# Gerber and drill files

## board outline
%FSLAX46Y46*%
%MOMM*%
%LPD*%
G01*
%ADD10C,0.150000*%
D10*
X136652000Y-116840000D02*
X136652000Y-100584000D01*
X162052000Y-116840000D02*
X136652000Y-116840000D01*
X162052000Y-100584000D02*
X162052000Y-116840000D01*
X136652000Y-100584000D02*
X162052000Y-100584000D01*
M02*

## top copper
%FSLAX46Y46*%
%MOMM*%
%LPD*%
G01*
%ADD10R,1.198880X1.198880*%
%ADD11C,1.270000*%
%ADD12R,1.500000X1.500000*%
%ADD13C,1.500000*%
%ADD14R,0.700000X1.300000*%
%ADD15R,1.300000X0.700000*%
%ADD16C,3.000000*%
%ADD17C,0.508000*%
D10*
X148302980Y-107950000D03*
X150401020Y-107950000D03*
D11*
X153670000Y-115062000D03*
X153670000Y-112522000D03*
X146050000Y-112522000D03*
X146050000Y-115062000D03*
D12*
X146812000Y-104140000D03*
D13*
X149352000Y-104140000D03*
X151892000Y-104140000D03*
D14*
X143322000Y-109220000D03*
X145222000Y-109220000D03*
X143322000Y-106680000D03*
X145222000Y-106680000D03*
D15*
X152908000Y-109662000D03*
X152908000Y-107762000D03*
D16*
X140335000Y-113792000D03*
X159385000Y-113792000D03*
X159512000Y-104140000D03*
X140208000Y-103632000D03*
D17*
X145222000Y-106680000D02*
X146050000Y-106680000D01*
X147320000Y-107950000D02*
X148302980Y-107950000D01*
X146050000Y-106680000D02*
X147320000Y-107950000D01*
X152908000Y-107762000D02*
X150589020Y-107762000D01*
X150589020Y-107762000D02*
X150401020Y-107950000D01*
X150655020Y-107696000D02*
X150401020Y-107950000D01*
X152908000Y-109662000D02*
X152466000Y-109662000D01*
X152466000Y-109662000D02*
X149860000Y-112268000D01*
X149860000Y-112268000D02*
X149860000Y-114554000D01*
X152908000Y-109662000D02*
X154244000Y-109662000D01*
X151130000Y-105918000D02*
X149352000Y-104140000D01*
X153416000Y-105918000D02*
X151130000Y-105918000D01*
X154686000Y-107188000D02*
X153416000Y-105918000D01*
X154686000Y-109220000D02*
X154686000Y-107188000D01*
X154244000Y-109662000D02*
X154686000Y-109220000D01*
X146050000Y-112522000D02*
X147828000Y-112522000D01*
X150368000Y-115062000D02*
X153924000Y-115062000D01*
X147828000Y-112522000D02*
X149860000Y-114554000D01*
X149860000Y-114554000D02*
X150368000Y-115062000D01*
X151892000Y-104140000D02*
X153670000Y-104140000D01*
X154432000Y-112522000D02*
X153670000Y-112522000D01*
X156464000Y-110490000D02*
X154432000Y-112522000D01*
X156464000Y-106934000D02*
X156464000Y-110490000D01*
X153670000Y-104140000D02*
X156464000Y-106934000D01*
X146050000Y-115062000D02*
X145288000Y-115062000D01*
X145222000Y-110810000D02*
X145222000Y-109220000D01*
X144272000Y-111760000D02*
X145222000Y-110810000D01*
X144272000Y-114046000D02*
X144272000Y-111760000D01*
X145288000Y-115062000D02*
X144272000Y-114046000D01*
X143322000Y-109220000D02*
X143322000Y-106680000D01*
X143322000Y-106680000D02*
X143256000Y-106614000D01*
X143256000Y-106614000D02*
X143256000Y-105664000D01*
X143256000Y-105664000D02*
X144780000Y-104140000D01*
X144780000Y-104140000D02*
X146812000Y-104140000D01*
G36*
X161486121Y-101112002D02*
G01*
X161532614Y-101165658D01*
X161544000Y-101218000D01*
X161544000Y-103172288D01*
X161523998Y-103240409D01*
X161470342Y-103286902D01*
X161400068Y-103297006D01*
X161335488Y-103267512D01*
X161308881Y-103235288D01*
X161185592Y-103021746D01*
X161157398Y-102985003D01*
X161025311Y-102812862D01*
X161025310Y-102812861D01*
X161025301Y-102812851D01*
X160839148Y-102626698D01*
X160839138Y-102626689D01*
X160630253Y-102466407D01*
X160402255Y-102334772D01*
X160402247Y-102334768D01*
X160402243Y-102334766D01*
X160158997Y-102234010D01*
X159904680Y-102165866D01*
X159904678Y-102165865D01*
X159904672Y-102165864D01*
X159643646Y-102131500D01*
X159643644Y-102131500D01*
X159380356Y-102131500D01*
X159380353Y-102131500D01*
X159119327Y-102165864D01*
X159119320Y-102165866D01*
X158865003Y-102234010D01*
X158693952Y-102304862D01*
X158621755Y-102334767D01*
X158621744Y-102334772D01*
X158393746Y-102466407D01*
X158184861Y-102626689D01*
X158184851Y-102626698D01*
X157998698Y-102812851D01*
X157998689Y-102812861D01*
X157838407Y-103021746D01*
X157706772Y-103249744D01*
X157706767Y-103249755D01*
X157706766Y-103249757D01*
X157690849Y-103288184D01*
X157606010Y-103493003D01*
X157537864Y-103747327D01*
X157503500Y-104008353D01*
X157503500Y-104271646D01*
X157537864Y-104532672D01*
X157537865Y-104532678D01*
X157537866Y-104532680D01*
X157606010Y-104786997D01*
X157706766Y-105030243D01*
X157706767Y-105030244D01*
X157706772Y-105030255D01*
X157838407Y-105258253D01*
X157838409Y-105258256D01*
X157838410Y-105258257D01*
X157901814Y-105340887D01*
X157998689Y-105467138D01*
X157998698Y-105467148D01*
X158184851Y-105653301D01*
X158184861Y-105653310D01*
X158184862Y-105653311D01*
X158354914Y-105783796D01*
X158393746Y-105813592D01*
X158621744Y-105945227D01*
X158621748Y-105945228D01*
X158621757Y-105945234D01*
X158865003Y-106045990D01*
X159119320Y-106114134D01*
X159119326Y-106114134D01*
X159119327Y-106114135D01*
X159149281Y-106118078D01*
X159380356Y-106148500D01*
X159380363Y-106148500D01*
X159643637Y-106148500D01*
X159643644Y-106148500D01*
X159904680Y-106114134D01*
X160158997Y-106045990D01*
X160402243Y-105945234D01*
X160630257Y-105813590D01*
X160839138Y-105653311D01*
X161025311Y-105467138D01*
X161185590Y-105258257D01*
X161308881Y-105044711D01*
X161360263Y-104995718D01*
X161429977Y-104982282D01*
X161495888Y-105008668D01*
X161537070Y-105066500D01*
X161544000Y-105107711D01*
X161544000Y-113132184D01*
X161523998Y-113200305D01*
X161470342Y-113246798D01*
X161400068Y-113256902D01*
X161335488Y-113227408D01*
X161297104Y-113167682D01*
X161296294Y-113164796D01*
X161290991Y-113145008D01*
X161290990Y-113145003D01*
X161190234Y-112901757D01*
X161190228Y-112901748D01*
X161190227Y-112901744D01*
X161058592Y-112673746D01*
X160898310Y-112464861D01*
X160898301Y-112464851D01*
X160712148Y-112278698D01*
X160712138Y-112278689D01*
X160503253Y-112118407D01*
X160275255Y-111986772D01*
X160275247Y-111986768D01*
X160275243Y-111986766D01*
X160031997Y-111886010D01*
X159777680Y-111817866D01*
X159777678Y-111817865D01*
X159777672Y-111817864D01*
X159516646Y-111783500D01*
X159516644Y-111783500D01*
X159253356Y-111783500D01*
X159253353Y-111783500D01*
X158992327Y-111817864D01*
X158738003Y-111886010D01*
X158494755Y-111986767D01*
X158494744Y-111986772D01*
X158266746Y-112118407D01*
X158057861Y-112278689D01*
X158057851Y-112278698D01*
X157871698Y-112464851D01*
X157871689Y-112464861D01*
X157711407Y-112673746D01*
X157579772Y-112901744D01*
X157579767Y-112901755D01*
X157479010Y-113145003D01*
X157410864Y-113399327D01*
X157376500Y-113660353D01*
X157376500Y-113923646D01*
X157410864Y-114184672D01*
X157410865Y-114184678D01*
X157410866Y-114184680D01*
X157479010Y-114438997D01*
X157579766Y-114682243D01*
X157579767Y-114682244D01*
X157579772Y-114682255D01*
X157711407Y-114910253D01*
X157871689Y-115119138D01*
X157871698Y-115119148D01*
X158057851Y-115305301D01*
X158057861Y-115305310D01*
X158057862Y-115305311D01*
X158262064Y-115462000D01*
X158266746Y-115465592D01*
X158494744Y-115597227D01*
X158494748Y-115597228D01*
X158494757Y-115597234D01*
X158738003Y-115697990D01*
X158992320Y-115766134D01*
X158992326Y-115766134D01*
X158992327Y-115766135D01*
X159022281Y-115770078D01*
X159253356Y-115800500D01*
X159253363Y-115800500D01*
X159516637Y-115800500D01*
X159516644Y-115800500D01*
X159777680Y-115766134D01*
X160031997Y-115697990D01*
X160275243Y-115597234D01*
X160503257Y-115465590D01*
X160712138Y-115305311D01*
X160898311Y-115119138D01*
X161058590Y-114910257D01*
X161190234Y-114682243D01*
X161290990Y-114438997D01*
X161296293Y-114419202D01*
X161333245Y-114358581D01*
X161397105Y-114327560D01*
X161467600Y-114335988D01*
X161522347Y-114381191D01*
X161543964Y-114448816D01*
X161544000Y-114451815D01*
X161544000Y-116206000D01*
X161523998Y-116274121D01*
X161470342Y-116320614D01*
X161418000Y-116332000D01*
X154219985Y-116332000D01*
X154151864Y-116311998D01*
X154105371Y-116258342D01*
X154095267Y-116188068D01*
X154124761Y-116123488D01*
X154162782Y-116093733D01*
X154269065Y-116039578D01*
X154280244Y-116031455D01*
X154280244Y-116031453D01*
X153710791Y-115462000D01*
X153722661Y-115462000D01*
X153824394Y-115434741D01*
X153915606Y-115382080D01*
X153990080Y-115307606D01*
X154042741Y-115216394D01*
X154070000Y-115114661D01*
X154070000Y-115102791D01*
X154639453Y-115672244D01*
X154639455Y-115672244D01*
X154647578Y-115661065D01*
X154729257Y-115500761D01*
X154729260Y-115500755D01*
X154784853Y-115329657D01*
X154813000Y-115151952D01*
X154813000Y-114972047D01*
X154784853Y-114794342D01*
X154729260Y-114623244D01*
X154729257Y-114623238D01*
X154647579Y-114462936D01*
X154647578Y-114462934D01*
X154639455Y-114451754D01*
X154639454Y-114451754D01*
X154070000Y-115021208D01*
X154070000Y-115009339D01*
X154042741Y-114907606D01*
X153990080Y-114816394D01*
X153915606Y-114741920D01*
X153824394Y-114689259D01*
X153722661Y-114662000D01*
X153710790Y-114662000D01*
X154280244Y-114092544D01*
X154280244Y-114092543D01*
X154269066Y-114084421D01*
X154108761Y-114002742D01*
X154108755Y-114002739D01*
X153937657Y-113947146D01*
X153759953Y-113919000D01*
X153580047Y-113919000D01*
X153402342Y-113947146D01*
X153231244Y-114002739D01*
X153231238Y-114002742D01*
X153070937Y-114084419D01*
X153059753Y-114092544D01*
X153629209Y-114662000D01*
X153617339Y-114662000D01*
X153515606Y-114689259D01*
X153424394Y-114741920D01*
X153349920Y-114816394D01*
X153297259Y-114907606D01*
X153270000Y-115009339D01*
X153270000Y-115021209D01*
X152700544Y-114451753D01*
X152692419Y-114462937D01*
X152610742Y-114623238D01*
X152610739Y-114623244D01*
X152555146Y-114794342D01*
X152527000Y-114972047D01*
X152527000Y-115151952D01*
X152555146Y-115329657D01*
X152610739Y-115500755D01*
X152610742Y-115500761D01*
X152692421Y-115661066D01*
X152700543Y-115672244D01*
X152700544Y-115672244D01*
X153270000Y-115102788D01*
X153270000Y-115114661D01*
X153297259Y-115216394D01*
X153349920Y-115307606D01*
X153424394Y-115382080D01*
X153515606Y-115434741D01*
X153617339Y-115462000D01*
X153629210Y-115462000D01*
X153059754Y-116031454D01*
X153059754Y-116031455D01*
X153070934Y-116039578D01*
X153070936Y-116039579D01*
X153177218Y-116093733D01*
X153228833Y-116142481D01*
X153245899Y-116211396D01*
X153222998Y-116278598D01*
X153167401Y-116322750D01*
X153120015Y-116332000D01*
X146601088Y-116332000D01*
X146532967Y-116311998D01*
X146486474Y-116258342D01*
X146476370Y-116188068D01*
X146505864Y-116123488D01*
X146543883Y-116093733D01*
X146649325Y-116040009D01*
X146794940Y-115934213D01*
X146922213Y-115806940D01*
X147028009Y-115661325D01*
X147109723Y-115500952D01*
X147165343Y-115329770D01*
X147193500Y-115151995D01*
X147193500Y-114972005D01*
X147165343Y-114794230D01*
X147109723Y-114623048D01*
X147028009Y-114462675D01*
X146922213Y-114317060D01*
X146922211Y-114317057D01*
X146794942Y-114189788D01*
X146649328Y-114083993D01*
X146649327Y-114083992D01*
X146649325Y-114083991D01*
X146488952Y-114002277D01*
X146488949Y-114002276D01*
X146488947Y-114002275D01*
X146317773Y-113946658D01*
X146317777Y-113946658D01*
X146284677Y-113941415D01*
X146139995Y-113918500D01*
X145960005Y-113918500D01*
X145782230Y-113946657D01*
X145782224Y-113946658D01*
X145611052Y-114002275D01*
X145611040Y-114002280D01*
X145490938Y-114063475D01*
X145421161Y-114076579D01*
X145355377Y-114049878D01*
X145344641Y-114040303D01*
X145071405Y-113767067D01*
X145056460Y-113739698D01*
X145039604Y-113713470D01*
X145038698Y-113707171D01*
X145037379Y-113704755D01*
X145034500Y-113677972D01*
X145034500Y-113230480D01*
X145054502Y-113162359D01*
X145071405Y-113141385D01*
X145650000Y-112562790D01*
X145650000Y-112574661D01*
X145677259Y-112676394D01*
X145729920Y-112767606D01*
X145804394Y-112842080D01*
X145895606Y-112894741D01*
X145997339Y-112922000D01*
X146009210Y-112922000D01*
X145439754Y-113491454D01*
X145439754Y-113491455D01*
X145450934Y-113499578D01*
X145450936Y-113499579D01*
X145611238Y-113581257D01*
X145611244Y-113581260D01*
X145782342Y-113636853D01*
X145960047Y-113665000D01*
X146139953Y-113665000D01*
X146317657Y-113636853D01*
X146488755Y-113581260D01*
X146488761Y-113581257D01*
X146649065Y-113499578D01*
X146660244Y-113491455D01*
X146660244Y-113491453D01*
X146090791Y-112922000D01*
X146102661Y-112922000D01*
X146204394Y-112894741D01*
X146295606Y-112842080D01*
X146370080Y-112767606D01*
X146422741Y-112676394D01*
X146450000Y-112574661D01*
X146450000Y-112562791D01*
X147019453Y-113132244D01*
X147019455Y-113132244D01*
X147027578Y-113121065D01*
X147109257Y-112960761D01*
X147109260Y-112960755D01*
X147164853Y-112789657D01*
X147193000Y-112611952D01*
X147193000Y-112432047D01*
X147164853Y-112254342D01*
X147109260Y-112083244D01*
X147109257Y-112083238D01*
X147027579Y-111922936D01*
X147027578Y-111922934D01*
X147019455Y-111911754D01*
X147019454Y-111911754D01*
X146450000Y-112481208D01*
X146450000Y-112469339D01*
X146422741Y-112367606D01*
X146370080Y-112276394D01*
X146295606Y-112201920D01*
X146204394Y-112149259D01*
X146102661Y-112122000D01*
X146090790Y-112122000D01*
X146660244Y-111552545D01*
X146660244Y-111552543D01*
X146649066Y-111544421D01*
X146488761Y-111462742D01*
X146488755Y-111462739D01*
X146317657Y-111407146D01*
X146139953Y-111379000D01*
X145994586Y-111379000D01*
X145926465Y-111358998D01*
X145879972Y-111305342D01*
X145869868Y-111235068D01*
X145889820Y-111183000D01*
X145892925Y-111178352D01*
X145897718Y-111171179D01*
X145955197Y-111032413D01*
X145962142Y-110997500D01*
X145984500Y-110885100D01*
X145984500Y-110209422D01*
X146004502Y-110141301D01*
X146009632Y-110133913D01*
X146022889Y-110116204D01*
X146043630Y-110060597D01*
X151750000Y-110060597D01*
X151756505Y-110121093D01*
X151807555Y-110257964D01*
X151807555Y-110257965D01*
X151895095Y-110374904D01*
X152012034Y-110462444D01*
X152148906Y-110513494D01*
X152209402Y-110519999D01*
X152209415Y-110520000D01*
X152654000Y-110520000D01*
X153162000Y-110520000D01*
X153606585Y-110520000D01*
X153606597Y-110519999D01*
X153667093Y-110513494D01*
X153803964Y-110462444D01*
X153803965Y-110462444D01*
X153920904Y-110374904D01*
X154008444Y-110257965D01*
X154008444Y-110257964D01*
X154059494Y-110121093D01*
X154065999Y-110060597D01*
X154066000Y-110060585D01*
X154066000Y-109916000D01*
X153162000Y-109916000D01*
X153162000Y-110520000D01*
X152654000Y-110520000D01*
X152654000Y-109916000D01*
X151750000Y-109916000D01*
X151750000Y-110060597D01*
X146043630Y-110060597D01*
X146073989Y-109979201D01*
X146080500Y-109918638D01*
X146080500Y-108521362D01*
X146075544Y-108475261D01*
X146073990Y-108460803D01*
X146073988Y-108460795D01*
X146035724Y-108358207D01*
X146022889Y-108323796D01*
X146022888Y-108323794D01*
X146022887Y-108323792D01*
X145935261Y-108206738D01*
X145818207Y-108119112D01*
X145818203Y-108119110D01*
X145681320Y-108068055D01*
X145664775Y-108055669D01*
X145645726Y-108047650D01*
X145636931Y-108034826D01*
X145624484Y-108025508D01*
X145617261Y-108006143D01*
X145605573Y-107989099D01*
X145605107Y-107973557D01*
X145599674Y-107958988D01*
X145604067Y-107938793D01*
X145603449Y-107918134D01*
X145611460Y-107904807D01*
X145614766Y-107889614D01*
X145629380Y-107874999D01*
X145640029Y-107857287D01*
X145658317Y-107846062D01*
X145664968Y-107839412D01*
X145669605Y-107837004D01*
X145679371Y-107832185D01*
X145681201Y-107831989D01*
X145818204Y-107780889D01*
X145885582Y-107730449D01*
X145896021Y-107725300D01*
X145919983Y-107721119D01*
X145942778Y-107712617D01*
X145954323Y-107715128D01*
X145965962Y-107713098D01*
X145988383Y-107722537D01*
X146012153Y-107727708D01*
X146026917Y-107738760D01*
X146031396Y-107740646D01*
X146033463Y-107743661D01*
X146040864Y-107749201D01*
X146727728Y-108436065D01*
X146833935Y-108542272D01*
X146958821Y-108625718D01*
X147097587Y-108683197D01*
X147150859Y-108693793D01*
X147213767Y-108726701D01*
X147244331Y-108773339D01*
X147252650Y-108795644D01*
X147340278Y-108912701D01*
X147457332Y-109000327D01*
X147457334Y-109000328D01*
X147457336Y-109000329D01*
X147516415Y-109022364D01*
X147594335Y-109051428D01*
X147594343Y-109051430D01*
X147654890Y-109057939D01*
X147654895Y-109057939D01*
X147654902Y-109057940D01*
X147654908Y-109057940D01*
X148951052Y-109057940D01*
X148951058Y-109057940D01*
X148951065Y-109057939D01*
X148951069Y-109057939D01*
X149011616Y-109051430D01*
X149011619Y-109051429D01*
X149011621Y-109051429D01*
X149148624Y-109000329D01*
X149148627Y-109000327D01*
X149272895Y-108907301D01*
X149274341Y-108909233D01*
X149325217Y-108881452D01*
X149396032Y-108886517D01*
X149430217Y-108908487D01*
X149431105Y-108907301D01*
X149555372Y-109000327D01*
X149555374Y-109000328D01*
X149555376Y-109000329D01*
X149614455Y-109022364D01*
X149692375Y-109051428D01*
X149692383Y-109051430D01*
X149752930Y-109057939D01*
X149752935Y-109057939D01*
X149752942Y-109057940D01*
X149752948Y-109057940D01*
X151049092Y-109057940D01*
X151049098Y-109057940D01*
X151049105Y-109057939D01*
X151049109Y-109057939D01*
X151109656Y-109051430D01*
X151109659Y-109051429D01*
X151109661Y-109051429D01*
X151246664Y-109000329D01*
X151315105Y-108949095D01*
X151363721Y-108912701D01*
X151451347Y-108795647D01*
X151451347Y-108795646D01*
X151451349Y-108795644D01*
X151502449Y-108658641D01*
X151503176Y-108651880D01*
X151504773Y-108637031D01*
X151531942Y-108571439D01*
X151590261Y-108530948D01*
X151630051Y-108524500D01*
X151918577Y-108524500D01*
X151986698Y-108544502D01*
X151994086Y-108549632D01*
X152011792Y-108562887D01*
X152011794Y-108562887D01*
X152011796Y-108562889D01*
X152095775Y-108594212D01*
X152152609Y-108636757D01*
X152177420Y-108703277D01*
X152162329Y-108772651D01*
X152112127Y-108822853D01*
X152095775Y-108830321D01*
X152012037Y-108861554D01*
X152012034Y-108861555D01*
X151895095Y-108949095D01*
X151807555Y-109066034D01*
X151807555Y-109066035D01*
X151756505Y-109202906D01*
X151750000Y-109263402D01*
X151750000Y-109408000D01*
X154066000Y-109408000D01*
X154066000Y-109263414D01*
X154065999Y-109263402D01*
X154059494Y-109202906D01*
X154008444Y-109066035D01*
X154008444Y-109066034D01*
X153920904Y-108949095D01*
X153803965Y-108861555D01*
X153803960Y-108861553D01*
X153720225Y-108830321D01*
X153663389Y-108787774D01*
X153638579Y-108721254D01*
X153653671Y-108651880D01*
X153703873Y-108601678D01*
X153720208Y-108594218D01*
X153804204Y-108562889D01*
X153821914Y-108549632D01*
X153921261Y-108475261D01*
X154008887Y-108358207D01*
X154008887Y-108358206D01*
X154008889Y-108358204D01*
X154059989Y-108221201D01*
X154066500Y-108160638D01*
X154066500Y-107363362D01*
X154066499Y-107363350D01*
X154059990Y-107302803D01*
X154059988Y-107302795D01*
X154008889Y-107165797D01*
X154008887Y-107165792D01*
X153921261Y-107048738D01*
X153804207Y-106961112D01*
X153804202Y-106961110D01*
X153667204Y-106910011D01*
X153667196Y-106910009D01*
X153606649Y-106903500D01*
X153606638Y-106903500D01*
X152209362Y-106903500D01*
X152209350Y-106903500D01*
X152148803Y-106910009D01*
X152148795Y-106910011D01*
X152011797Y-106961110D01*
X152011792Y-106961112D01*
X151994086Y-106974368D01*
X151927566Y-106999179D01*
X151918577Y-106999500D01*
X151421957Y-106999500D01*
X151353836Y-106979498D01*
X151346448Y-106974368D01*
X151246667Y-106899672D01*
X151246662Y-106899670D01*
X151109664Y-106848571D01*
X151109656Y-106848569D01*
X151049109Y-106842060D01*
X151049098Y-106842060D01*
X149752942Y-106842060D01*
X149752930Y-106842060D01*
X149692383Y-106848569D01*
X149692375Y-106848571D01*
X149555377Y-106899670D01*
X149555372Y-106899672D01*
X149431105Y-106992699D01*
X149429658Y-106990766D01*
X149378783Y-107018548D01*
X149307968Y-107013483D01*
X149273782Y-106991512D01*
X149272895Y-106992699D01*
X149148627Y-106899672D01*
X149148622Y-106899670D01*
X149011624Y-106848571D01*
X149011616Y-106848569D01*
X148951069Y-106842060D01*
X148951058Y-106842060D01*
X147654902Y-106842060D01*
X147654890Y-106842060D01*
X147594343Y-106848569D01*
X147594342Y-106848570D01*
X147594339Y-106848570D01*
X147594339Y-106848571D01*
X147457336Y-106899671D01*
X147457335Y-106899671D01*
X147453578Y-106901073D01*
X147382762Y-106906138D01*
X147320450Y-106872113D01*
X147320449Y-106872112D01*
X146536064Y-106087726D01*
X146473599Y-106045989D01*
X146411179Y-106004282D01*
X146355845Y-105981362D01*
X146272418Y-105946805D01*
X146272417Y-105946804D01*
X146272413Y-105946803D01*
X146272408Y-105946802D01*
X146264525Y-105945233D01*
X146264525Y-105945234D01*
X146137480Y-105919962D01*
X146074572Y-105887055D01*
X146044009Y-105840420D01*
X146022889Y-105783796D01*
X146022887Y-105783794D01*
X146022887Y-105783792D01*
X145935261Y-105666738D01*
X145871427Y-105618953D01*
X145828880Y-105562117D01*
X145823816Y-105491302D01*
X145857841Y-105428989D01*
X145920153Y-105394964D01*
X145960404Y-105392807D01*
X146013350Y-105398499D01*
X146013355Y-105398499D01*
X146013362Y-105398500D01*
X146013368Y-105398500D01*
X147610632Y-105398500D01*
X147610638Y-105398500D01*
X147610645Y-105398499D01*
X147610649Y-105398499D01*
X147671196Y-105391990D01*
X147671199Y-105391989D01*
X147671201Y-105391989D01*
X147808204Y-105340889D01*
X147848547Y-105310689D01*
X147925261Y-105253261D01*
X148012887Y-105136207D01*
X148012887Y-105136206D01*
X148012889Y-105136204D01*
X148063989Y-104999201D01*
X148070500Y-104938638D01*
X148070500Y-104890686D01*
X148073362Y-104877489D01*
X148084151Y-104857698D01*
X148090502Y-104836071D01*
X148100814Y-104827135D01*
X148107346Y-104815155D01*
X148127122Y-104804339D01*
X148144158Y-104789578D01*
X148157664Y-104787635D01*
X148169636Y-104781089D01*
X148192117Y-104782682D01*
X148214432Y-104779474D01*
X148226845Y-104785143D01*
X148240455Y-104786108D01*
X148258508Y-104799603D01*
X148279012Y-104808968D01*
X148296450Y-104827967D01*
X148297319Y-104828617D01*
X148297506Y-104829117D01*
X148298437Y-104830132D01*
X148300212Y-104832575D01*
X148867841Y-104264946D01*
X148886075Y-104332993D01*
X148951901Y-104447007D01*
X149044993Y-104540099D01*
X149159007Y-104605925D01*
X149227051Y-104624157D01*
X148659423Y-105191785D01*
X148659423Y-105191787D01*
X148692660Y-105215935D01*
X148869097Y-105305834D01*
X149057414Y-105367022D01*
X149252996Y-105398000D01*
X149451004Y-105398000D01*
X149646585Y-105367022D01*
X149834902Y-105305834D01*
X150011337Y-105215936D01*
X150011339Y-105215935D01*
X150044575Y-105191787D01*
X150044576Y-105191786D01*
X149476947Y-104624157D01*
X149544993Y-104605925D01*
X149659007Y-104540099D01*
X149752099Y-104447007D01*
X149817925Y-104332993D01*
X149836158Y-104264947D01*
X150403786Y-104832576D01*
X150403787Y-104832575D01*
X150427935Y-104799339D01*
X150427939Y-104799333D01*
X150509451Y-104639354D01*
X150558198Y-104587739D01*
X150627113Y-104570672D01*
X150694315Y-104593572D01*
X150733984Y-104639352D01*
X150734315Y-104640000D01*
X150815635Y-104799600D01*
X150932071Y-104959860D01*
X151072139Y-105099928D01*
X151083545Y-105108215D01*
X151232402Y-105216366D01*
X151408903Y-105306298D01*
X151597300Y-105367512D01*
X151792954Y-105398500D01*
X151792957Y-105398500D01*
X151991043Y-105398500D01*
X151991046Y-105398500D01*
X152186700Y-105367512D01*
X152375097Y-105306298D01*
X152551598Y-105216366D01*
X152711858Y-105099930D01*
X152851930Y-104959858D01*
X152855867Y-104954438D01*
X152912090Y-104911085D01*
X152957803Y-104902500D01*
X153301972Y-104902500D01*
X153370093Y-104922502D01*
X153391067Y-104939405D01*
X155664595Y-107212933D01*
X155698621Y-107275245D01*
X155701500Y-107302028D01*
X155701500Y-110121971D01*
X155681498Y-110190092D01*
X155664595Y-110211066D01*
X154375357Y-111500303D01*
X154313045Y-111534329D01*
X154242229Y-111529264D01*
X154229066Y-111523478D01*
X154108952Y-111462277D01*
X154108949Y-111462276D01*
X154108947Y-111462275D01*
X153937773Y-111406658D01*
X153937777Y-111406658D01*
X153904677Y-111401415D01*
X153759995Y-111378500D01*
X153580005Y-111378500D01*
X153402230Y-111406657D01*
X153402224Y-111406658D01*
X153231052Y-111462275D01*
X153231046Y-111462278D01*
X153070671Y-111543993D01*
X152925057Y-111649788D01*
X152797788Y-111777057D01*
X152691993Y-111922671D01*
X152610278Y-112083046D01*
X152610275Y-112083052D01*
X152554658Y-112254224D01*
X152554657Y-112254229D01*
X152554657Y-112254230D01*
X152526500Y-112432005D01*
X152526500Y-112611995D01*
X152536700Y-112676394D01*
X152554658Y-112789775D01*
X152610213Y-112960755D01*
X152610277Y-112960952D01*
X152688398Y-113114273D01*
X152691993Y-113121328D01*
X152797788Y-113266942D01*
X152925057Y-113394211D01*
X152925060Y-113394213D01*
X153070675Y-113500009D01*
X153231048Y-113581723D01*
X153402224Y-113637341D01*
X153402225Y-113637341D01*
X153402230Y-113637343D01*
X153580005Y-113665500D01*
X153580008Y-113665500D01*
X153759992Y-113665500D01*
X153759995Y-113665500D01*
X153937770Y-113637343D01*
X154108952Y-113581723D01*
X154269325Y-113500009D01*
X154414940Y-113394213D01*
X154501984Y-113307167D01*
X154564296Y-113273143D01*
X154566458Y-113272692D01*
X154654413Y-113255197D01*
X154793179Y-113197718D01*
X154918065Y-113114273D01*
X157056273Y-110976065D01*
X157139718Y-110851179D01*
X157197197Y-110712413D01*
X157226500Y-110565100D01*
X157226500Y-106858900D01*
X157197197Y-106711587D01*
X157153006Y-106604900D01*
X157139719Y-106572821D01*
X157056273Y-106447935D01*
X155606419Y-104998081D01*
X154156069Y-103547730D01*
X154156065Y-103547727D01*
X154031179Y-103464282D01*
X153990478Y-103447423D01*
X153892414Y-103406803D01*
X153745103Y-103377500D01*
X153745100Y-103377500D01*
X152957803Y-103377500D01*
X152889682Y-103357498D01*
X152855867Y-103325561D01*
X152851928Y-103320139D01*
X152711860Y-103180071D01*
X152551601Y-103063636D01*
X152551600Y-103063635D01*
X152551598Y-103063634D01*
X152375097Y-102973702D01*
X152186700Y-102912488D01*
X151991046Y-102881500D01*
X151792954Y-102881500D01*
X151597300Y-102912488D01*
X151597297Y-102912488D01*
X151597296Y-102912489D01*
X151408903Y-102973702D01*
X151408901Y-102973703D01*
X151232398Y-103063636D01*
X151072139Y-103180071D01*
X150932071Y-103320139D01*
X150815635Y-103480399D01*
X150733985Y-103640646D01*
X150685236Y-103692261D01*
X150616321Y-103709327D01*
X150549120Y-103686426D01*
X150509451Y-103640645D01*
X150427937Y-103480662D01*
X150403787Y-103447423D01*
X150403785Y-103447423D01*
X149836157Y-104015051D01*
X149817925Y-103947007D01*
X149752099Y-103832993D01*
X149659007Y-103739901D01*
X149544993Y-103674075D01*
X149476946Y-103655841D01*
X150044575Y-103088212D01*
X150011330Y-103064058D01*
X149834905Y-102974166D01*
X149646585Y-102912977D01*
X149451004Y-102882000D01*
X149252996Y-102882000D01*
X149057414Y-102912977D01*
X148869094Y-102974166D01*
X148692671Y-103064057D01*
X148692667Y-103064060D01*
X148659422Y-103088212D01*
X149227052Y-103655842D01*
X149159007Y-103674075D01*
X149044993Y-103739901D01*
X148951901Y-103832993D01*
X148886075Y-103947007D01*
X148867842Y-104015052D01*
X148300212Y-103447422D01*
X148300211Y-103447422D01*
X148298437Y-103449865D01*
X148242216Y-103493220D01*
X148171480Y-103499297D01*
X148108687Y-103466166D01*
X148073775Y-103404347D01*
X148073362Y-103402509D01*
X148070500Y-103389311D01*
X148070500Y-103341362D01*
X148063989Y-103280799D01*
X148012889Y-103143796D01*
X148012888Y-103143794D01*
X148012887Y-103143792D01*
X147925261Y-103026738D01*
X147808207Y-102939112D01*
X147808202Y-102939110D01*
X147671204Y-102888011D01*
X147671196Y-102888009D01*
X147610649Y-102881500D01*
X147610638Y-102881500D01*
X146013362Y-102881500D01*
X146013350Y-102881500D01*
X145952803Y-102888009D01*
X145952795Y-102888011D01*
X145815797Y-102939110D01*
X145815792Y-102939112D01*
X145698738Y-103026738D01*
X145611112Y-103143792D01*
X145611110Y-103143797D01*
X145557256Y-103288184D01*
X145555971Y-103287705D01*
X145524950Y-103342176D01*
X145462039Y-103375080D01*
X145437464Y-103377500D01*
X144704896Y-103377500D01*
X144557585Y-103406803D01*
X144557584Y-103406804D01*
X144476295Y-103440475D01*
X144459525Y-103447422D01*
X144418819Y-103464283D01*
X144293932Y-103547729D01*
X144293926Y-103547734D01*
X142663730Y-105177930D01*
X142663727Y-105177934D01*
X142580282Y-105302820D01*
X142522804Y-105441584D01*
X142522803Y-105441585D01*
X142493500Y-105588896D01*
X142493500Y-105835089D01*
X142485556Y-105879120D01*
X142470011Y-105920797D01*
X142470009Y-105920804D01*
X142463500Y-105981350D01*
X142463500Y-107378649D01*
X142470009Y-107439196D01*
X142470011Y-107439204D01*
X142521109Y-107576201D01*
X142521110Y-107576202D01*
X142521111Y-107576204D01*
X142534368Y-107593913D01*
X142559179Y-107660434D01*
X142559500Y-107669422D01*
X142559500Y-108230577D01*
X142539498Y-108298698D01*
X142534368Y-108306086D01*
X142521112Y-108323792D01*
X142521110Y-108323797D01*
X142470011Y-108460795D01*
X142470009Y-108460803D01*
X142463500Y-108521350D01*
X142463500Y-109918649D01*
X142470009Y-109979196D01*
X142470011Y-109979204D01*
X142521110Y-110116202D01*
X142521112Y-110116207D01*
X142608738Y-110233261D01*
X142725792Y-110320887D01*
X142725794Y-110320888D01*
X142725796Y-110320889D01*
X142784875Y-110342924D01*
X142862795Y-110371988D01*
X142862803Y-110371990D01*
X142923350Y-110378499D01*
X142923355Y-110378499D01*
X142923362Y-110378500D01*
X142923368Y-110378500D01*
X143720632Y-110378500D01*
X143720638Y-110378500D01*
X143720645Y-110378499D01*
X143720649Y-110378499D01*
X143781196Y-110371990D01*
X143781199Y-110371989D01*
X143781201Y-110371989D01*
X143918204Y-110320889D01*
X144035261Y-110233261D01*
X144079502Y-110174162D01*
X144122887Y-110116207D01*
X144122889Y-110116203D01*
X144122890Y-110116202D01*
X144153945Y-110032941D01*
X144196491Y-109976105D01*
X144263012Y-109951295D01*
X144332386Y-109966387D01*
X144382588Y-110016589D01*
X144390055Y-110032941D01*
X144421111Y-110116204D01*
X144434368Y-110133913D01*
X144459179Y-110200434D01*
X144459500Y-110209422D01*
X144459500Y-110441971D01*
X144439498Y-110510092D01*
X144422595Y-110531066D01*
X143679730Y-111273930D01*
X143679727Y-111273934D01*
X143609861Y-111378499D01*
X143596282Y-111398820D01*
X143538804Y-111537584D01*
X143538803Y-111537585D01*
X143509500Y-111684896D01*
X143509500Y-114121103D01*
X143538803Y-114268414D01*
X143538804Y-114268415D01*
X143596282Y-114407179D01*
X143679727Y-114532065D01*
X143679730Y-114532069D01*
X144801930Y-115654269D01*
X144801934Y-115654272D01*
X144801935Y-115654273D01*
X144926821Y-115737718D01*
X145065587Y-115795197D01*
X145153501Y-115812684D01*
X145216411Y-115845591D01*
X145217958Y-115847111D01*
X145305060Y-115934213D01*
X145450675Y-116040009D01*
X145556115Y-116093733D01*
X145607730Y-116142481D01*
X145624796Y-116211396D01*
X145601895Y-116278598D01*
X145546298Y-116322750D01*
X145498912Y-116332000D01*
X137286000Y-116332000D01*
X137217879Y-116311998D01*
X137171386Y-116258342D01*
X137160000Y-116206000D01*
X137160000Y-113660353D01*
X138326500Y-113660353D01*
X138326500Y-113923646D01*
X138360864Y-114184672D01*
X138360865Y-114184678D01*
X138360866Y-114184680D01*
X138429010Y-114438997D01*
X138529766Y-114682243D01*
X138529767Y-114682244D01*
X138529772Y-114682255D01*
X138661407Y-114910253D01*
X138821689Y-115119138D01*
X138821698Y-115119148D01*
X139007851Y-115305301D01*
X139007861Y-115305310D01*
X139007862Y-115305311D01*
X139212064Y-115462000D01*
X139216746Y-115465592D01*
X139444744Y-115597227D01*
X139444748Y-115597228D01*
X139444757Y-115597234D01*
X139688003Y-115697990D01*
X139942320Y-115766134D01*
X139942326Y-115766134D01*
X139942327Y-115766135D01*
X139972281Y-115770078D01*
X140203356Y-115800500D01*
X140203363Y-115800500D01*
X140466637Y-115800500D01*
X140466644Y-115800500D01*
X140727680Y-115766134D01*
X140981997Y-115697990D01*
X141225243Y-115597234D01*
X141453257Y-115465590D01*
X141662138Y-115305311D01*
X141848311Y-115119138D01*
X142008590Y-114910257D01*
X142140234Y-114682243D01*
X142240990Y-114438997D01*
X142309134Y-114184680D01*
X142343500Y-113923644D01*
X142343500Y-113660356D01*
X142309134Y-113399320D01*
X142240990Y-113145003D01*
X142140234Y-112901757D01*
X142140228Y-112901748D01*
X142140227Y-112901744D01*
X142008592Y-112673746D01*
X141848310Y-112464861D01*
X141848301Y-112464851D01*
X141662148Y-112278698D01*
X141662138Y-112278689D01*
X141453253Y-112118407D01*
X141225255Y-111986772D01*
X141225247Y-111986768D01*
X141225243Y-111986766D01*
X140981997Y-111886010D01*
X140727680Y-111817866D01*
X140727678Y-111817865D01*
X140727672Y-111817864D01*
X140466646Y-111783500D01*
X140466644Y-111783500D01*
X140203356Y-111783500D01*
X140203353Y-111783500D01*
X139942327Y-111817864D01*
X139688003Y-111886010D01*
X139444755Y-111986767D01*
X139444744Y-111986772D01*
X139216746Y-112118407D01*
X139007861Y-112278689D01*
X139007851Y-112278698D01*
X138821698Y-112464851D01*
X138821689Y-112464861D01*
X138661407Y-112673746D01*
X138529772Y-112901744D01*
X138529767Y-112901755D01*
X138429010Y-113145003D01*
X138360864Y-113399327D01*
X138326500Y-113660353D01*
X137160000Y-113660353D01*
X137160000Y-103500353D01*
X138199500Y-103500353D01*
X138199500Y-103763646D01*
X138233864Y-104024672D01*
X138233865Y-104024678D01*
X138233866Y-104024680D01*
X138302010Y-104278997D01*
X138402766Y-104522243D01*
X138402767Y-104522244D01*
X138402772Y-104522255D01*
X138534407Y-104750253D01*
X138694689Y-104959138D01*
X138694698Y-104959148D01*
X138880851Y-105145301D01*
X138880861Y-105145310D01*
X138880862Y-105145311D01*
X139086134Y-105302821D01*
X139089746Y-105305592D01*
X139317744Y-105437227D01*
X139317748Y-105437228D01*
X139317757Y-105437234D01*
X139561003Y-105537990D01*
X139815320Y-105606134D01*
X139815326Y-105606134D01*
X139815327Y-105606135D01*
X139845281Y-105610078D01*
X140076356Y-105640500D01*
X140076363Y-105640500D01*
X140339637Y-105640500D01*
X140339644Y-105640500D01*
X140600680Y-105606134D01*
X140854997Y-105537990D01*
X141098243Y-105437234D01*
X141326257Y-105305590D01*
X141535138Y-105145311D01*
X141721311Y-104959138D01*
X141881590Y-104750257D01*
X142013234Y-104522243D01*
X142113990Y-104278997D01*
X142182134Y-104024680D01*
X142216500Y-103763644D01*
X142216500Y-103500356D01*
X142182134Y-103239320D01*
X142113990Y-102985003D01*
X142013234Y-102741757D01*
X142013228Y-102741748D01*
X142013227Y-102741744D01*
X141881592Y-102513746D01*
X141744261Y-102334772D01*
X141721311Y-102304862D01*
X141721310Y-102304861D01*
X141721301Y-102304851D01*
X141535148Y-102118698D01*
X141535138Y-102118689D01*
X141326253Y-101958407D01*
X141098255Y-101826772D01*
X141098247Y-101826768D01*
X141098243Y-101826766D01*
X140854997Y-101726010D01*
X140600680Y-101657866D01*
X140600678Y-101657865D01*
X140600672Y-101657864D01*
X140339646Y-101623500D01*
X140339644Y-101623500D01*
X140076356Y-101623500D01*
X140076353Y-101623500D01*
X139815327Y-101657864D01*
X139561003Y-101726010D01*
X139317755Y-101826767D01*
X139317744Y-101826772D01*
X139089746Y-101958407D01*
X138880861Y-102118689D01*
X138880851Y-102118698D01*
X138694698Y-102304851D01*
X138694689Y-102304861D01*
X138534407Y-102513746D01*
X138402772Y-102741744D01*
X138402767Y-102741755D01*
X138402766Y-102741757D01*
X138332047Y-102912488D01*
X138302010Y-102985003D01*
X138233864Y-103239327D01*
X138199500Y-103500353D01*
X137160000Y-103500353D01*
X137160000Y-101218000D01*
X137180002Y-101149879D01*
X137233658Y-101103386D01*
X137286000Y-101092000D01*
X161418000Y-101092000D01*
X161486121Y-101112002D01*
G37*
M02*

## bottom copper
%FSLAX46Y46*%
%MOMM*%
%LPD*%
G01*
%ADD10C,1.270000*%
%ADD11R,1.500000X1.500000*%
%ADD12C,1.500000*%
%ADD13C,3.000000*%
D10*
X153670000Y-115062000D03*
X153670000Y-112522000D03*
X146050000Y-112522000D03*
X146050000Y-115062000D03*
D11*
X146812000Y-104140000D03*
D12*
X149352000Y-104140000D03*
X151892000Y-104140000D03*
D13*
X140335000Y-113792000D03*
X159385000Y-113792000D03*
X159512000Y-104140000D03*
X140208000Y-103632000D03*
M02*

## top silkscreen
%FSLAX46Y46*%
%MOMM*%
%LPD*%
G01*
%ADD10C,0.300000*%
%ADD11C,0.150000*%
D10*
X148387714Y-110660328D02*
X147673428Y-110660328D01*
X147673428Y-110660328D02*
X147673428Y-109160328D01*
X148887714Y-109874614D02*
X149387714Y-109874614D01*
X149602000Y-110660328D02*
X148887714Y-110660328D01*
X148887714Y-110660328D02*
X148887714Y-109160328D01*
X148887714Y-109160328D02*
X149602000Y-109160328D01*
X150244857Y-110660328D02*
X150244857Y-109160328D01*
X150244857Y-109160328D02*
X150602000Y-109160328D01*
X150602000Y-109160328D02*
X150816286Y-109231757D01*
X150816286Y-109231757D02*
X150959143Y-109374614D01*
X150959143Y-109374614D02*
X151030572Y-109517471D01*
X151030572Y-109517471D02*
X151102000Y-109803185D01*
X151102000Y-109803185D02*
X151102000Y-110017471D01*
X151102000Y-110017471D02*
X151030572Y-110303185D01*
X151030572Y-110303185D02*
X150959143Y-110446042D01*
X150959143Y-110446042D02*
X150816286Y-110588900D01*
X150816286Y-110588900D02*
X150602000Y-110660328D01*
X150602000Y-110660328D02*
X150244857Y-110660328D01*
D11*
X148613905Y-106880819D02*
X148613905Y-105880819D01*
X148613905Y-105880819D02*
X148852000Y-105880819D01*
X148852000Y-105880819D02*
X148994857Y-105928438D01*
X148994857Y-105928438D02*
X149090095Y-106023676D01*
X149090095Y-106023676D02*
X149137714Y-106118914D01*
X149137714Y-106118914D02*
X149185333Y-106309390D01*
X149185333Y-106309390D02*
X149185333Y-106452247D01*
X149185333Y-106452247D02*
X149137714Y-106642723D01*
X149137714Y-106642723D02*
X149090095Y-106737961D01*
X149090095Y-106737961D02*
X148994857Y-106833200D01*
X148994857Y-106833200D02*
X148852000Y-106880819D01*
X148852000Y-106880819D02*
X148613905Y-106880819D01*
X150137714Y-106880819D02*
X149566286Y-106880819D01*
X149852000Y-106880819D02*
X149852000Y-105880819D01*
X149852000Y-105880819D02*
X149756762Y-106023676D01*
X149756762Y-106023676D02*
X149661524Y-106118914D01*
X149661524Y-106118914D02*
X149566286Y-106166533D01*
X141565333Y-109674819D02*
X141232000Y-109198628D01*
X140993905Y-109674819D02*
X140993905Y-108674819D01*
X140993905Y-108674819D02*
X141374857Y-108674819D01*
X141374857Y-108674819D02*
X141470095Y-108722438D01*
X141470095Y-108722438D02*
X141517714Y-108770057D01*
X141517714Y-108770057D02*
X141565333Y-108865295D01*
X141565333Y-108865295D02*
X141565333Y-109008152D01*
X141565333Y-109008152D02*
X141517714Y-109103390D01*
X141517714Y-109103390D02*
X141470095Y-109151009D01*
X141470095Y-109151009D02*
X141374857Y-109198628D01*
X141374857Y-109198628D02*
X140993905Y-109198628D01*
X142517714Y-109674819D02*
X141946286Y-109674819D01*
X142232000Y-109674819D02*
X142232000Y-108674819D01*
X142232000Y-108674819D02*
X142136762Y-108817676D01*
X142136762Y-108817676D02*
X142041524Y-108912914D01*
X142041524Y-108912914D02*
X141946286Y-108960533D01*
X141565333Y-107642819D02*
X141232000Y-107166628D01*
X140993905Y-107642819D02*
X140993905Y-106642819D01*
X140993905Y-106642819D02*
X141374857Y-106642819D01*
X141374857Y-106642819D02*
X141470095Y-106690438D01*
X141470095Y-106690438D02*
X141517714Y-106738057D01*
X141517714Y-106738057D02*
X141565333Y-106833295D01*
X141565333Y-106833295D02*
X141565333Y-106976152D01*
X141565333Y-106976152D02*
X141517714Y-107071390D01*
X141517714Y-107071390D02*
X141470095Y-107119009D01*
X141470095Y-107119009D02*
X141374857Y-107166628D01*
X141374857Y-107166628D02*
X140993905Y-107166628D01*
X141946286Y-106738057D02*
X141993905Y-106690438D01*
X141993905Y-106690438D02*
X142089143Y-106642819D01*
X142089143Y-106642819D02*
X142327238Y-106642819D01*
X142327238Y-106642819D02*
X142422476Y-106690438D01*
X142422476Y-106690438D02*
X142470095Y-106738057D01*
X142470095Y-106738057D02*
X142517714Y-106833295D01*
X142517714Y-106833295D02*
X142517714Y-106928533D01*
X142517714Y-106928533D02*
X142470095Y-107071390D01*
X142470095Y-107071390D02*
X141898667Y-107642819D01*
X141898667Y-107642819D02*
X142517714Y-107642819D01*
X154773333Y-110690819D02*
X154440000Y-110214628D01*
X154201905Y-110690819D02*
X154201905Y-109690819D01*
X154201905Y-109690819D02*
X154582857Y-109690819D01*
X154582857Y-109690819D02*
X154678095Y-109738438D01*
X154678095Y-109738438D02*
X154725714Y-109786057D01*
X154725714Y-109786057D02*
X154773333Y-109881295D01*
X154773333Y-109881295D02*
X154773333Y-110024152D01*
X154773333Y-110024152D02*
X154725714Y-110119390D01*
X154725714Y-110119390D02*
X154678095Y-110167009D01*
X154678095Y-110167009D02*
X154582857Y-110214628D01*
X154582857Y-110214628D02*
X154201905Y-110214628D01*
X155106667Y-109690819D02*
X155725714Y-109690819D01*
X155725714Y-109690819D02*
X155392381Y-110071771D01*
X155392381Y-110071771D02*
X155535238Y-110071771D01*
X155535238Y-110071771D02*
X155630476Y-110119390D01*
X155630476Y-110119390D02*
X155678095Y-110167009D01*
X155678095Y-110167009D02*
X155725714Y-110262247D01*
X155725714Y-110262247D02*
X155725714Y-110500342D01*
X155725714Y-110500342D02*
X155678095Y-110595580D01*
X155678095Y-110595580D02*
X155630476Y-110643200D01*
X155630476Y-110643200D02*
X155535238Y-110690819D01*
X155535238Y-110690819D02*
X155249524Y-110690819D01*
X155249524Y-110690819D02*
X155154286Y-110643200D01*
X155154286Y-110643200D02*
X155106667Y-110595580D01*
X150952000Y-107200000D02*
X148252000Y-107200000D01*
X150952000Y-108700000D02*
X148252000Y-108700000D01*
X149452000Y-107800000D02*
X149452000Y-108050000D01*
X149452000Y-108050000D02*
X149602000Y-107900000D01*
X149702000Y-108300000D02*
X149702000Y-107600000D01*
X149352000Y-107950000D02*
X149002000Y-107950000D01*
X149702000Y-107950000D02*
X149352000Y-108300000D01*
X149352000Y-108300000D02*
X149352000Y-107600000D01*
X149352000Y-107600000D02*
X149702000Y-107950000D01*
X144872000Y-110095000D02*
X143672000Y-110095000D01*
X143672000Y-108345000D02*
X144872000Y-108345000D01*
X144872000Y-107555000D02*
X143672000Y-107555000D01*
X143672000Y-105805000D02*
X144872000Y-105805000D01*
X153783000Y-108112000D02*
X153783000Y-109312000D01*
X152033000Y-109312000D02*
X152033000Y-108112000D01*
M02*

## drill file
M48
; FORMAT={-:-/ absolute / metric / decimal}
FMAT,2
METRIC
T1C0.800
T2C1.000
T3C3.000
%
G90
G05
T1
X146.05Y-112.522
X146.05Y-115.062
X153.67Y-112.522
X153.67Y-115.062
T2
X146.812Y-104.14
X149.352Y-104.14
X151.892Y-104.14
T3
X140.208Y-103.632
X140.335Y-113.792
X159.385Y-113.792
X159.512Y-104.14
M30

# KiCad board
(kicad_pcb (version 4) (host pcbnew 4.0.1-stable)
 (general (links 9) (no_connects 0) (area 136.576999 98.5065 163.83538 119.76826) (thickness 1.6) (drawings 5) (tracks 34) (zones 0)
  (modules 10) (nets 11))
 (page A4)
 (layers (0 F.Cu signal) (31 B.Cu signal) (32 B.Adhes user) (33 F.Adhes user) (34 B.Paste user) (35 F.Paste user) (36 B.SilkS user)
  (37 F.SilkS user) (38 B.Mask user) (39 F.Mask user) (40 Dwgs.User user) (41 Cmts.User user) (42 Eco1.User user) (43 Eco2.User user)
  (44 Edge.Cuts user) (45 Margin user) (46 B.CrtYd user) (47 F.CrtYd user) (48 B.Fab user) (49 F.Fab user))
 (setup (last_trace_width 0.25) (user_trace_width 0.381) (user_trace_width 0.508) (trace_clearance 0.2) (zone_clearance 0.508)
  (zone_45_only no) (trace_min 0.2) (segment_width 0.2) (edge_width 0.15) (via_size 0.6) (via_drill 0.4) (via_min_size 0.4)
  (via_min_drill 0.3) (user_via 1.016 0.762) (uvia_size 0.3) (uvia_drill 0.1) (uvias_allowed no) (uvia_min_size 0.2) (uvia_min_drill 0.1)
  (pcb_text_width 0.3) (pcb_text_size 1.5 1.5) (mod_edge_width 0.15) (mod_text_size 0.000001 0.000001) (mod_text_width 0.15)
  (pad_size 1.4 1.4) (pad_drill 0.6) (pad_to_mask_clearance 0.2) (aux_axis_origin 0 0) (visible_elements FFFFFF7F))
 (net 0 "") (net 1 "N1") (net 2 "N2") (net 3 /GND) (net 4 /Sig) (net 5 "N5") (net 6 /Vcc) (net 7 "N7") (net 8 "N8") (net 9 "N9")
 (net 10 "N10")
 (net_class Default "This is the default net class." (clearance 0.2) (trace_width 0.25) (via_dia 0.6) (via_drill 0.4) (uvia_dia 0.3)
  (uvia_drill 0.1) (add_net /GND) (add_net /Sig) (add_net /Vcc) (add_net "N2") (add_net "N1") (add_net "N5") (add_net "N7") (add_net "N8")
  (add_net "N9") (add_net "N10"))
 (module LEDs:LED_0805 (layer F.Cu) (at 149.352 107.95 180)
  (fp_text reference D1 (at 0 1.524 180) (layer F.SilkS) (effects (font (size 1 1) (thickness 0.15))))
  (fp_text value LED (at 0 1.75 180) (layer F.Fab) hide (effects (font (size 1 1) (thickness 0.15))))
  (fp_line (start -1.6 0.75) (end 1.1 0.75) (layer F.SilkS) (width 0.15))
  (fp_line (start -1.6 -0.75) (end 1.1 -0.75) (layer F.SilkS) (width 0.15))
  (fp_line (start -0.1 0.15) (end -0.1 -0.1) (layer F.SilkS) (width 0.15))
  (fp_line (start -0.1 -0.1) (end -0.25 0.05) (layer F.SilkS) (width 0.15))
  (fp_line (start -0.35 -0.35) (end -0.35 0.35) (layer F.SilkS) (width 0.15))
  (fp_line (start 0 0) (end 0.35 0) (layer F.SilkS) (width 0.15))
  (fp_line (start -0.35 0) (end 0 -0.35) (layer F.SilkS) (width 0.15))
  (fp_line (start 0 -0.35) (end 0 0.35) (layer F.SilkS) (width 0.15))
  (fp_line (start 0 0.35) (end -0.35 0) (layer F.SilkS) (width 0.15))
  (pad 2 smd rect (at 1.04902 0) (size 1.19888 1.19888) (layers F.Cu F.Paste F.Mask) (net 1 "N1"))
  (pad 1 smd rect (at -1.04902 0) (size 1.19888 1.19888) (layers F.Cu F.Paste F.Mask) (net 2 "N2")))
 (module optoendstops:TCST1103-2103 (layer B.Cu) (at 149.86 113.792)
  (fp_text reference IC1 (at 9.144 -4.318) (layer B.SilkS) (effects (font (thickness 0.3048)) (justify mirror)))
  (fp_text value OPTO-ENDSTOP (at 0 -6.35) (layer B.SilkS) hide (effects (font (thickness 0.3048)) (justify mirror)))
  (pad E/D thru_hole circle (at 3.81 1.27) (size 1.27 1.27) (drill 0.8) (layers *.Cu *.Mask B.SilkS) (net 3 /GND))
  (pad C/+ thru_hole circle (at 3.81 -1.27) (size 1.27 1.27) (drill 0.8) (layers *.Cu *.Mask B.SilkS) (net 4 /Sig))
  (pad K/E thru_hole circle (at -3.81 -1.27) (size 1.27 1.27) (drill 0.8) (layers *.Cu *.Mask B.SilkS) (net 3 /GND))
  (pad A/+ thru_hole circle (at -3.81 1.27) (size 1.27 1.27) (drill 0.8) (layers *.Cu *.Mask B.SilkS) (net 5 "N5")))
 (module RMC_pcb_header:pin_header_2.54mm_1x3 (layer B.Cu) (at 149.352 104.14)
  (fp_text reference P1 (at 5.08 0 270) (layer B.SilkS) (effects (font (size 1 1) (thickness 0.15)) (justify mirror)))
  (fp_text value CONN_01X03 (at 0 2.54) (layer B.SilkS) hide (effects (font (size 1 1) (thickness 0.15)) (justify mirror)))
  (pad 1 thru_hole rect (at -2.54 0) (size 1.5 1.5) (drill 1) (layers *.Cu *.Mask B.SilkS) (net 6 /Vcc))
  (pad 2 thru_hole circle (at 0 0) (size 1.5 1.5) (drill 1) (layers *.Cu *.Mask B.SilkS) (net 3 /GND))
  (pad 3 thru_hole circle (at 2.54 0) (size 1.5 1.5) (drill 1) (layers *.Cu *.Mask B.SilkS) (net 4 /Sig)))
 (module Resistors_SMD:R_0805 (layer F.Cu) (at 144.272 109.22)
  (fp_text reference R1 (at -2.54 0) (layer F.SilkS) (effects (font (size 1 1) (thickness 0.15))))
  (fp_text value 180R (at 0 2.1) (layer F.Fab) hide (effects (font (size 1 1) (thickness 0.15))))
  (fp_line (start 0.6 0.875) (end -0.6 0.875) (layer F.SilkS) (width 0.15))
  (fp_line (start -0.6 -0.875) (end 0.6 -0.875) (layer F.SilkS) (width 0.15))
  (pad 1 smd rect (at -0.95 0) (size 0.7 1.3) (layers F.Cu F.Paste F.Mask) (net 6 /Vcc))
  (pad 2 smd rect (at 0.95 0) (size 0.7 1.3) (layers F.Cu F.Paste F.Mask) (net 5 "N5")))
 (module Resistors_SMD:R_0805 (layer F.Cu) (at 144.272 106.68)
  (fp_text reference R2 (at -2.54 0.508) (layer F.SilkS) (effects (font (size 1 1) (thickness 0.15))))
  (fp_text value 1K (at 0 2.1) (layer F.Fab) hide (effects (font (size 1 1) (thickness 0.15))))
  (fp_line (start 0.6 0.875) (end -0.6 0.875) (layer F.SilkS) (width 0.15))
  (fp_line (start -0.6 -0.875) (end 0.6 -0.875) (layer F.SilkS) (width 0.15))
  (pad 1 smd rect (at -0.95 0) (size 0.7 1.3) (layers F.Cu F.Paste F.Mask) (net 6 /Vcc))
  (pad 2 smd rect (at 0.95 0) (size 0.7 1.3) (layers F.Cu F.Paste F.Mask) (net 1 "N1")))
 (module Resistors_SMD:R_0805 (layer F.Cu) (at 152.908 108.712 90)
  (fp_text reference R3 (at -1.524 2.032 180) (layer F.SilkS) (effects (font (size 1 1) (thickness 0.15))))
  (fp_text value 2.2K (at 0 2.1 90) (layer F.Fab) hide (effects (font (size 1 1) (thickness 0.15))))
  (fp_line (start 0.6 0.875) (end -0.6 0.875) (layer F.SilkS) (width 0.15))
  (fp_line (start -0.6 -0.875) (end 0.6 -0.875) (layer F.SilkS) (width 0.15))
  (pad 1 smd rect (at -0.95 0 90) (size 0.7 1.3) (layers F.Cu F.Paste F.Mask) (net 3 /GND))
  (pad 2 smd rect (at 0.95 0 90) (size 0.7 1.3) (layers F.Cu F.Paste F.Mask) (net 2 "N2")))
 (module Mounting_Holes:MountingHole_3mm (layer F.Cu) (at 140.335 113.792)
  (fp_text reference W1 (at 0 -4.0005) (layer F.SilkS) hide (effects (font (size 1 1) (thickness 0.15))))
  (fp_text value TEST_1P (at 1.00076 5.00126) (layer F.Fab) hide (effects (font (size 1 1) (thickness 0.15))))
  (pad 1 thru_hole circle (at 0 0) (size 3 3) (drill 3) (layers) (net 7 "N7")))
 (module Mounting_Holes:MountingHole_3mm (layer F.Cu) (at 159.385 113.792)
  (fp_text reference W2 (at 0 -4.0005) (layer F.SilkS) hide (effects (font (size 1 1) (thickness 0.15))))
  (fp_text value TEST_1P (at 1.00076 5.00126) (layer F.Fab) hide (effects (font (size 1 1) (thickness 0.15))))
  (pad 1 thru_hole circle (at 0 0) (size 3 3) (drill 3) (layers) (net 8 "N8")))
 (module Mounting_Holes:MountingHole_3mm (layer F.Cu) (at 159.512 104.14)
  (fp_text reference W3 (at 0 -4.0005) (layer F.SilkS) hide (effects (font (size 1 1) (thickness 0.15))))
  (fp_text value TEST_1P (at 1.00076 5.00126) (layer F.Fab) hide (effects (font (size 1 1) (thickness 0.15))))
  (pad 1 thru_hole circle (at 0 0) (size 3 3) (drill 3) (layers) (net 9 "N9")))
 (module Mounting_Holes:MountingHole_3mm (layer F.Cu) (at 140.208 103.632)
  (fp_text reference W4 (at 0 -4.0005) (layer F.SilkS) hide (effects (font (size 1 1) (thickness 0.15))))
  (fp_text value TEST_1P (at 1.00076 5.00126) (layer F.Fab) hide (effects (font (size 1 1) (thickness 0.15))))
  (pad 1 thru_hole circle (at 0 0) (size 3 3) (drill 3) (layers) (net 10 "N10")))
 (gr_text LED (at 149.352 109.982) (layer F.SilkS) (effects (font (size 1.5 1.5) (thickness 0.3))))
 (gr_line (start 136.652 116.84) (end 136.652 100.584) (angle 90) (layer Edge.Cuts) (width 0.15))
 (gr_line (start 162.052 116.84) (end 136.652 116.84) (angle 90) (layer Edge.Cuts) (width 0.15))
 (gr_line (start 162.052 100.584) (end 162.052 116.84) (angle 90) (layer Edge.Cuts) (width 0.15))
 (gr_line (start 136.652 100.584) (end 162.052 100.584) (angle 90) (layer Edge.Cuts) (width 0.15))
 (segment (start 145.222 106.68) (end 146.05 106.68) (width 0.508) (layer F.Cu) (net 1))
 (segment (start 147.32 107.95) (end 148.30298 107.95) (width 0.508) (layer F.Cu) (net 1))
 (segment (start 146.05 106.68) (end 147.32 107.95) (width 0.508) (layer F.Cu) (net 1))
 (segment (start 152.908 107.762) (end 150.58902 107.762) (width 0.508) (layer F.Cu) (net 2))
 (segment (start 150.58902 107.762) (end 150.40102 107.95) (width 0.508) (layer F.Cu) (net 2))
 (segment (start 150.65502 107.696) (end 150.40102 107.95) (width 0.508) (layer F.Cu) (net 2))
 (segment (start 152.908 109.662) (end 152.466 109.662) (width 0.508) (layer F.Cu) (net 3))
 (segment (start 152.466 109.662) (end 149.86 112.268) (width 0.508) (layer F.Cu) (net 3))
 (segment (start 149.86 112.268) (end 149.86 114.554) (width 0.508) (layer F.Cu) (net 3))
 (segment (start 152.908 109.662) (end 154.244 109.662) (width 0.508) (layer F.Cu) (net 3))
 (segment (start 151.13 105.918) (end 149.352 104.14) (width 0.508) (layer F.Cu) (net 3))
 (segment (start 153.416 105.918) (end 151.13 105.918) (width 0.508) (layer F.Cu) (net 3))
 (segment (start 154.686 107.188) (end 153.416 105.918) (width 0.508) (layer F.Cu) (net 3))
 (segment (start 154.686 109.22) (end 154.686 107.188) (width 0.508) (layer F.Cu) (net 3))
 (segment (start 154.244 109.662) (end 154.686 109.22) (width 0.508) (layer F.Cu) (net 3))
 (segment (start 146.05 112.522) (end 147.828 112.522) (width 0.508) (layer F.Cu) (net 3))
 (segment (start 150.368 115.062) (end 153.924 115.062) (width 0.508) (layer F.Cu) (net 3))
 (segment (start 147.828 112.522) (end 149.86 114.554) (width 0.508) (layer F.Cu) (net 3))
 (segment (start 149.86 114.554) (end 150.368 115.062) (width 0.508) (layer F.Cu) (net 3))
 (segment (start 151.892 104.14) (end 153.67 104.14) (width 0.508) (layer F.Cu) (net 4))
 (segment (start 154.432 112.522) (end 153.67 112.522) (width 0.508) (layer F.Cu) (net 4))
 (segment (start 156.464 110.49) (end 154.432 112.522) (width 0.508) (layer F.Cu) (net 4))
 (segment (start 156.464 106.934) (end 156.464 110.49) (width 0.508) (layer F.Cu) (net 4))
 (segment (start 153.67 104.14) (end 156.464 106.934) (width 0.508) (layer F.Cu) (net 4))
 (segment (start 146.05 115.062) (end 145.288 115.062) (width 0.508) (layer F.Cu) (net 5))
 (segment (start 145.222 110.81) (end 145.222 109.22) (width 0.508) (layer F.Cu) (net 5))
 (segment (start 144.272 111.76) (end 145.222 110.81) (width 0.508) (layer F.Cu) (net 5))
 (segment (start 144.272 114.046) (end 144.272 111.76) (width 0.508) (layer F.Cu) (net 5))
 (segment (start 145.288 115.062) (end 144.272 114.046) (width 0.508) (layer F.Cu) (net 5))
 (segment (start 143.322 109.22) (end 143.322 106.68) (width 0.508) (layer F.Cu) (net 6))
 (segment (start 143.322 106.68) (end 143.256 106.614) (width 0.508) (layer F.Cu) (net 6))
 (segment (start 143.256 106.614) (end 143.256 105.664) (width 0.508) (layer F.Cu) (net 6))
 (segment (start 143.256 105.664) (end 144.78 104.14) (width 0.508) (layer F.Cu) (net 6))
 (segment (start 144.78 104.14) (end 146.812 104.14) (width 0.508) (layer F.Cu) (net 6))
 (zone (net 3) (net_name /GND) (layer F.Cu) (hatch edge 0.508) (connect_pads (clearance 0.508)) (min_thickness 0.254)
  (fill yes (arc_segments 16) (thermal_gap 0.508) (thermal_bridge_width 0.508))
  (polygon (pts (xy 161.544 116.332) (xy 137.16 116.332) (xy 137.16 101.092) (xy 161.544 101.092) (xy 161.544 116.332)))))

